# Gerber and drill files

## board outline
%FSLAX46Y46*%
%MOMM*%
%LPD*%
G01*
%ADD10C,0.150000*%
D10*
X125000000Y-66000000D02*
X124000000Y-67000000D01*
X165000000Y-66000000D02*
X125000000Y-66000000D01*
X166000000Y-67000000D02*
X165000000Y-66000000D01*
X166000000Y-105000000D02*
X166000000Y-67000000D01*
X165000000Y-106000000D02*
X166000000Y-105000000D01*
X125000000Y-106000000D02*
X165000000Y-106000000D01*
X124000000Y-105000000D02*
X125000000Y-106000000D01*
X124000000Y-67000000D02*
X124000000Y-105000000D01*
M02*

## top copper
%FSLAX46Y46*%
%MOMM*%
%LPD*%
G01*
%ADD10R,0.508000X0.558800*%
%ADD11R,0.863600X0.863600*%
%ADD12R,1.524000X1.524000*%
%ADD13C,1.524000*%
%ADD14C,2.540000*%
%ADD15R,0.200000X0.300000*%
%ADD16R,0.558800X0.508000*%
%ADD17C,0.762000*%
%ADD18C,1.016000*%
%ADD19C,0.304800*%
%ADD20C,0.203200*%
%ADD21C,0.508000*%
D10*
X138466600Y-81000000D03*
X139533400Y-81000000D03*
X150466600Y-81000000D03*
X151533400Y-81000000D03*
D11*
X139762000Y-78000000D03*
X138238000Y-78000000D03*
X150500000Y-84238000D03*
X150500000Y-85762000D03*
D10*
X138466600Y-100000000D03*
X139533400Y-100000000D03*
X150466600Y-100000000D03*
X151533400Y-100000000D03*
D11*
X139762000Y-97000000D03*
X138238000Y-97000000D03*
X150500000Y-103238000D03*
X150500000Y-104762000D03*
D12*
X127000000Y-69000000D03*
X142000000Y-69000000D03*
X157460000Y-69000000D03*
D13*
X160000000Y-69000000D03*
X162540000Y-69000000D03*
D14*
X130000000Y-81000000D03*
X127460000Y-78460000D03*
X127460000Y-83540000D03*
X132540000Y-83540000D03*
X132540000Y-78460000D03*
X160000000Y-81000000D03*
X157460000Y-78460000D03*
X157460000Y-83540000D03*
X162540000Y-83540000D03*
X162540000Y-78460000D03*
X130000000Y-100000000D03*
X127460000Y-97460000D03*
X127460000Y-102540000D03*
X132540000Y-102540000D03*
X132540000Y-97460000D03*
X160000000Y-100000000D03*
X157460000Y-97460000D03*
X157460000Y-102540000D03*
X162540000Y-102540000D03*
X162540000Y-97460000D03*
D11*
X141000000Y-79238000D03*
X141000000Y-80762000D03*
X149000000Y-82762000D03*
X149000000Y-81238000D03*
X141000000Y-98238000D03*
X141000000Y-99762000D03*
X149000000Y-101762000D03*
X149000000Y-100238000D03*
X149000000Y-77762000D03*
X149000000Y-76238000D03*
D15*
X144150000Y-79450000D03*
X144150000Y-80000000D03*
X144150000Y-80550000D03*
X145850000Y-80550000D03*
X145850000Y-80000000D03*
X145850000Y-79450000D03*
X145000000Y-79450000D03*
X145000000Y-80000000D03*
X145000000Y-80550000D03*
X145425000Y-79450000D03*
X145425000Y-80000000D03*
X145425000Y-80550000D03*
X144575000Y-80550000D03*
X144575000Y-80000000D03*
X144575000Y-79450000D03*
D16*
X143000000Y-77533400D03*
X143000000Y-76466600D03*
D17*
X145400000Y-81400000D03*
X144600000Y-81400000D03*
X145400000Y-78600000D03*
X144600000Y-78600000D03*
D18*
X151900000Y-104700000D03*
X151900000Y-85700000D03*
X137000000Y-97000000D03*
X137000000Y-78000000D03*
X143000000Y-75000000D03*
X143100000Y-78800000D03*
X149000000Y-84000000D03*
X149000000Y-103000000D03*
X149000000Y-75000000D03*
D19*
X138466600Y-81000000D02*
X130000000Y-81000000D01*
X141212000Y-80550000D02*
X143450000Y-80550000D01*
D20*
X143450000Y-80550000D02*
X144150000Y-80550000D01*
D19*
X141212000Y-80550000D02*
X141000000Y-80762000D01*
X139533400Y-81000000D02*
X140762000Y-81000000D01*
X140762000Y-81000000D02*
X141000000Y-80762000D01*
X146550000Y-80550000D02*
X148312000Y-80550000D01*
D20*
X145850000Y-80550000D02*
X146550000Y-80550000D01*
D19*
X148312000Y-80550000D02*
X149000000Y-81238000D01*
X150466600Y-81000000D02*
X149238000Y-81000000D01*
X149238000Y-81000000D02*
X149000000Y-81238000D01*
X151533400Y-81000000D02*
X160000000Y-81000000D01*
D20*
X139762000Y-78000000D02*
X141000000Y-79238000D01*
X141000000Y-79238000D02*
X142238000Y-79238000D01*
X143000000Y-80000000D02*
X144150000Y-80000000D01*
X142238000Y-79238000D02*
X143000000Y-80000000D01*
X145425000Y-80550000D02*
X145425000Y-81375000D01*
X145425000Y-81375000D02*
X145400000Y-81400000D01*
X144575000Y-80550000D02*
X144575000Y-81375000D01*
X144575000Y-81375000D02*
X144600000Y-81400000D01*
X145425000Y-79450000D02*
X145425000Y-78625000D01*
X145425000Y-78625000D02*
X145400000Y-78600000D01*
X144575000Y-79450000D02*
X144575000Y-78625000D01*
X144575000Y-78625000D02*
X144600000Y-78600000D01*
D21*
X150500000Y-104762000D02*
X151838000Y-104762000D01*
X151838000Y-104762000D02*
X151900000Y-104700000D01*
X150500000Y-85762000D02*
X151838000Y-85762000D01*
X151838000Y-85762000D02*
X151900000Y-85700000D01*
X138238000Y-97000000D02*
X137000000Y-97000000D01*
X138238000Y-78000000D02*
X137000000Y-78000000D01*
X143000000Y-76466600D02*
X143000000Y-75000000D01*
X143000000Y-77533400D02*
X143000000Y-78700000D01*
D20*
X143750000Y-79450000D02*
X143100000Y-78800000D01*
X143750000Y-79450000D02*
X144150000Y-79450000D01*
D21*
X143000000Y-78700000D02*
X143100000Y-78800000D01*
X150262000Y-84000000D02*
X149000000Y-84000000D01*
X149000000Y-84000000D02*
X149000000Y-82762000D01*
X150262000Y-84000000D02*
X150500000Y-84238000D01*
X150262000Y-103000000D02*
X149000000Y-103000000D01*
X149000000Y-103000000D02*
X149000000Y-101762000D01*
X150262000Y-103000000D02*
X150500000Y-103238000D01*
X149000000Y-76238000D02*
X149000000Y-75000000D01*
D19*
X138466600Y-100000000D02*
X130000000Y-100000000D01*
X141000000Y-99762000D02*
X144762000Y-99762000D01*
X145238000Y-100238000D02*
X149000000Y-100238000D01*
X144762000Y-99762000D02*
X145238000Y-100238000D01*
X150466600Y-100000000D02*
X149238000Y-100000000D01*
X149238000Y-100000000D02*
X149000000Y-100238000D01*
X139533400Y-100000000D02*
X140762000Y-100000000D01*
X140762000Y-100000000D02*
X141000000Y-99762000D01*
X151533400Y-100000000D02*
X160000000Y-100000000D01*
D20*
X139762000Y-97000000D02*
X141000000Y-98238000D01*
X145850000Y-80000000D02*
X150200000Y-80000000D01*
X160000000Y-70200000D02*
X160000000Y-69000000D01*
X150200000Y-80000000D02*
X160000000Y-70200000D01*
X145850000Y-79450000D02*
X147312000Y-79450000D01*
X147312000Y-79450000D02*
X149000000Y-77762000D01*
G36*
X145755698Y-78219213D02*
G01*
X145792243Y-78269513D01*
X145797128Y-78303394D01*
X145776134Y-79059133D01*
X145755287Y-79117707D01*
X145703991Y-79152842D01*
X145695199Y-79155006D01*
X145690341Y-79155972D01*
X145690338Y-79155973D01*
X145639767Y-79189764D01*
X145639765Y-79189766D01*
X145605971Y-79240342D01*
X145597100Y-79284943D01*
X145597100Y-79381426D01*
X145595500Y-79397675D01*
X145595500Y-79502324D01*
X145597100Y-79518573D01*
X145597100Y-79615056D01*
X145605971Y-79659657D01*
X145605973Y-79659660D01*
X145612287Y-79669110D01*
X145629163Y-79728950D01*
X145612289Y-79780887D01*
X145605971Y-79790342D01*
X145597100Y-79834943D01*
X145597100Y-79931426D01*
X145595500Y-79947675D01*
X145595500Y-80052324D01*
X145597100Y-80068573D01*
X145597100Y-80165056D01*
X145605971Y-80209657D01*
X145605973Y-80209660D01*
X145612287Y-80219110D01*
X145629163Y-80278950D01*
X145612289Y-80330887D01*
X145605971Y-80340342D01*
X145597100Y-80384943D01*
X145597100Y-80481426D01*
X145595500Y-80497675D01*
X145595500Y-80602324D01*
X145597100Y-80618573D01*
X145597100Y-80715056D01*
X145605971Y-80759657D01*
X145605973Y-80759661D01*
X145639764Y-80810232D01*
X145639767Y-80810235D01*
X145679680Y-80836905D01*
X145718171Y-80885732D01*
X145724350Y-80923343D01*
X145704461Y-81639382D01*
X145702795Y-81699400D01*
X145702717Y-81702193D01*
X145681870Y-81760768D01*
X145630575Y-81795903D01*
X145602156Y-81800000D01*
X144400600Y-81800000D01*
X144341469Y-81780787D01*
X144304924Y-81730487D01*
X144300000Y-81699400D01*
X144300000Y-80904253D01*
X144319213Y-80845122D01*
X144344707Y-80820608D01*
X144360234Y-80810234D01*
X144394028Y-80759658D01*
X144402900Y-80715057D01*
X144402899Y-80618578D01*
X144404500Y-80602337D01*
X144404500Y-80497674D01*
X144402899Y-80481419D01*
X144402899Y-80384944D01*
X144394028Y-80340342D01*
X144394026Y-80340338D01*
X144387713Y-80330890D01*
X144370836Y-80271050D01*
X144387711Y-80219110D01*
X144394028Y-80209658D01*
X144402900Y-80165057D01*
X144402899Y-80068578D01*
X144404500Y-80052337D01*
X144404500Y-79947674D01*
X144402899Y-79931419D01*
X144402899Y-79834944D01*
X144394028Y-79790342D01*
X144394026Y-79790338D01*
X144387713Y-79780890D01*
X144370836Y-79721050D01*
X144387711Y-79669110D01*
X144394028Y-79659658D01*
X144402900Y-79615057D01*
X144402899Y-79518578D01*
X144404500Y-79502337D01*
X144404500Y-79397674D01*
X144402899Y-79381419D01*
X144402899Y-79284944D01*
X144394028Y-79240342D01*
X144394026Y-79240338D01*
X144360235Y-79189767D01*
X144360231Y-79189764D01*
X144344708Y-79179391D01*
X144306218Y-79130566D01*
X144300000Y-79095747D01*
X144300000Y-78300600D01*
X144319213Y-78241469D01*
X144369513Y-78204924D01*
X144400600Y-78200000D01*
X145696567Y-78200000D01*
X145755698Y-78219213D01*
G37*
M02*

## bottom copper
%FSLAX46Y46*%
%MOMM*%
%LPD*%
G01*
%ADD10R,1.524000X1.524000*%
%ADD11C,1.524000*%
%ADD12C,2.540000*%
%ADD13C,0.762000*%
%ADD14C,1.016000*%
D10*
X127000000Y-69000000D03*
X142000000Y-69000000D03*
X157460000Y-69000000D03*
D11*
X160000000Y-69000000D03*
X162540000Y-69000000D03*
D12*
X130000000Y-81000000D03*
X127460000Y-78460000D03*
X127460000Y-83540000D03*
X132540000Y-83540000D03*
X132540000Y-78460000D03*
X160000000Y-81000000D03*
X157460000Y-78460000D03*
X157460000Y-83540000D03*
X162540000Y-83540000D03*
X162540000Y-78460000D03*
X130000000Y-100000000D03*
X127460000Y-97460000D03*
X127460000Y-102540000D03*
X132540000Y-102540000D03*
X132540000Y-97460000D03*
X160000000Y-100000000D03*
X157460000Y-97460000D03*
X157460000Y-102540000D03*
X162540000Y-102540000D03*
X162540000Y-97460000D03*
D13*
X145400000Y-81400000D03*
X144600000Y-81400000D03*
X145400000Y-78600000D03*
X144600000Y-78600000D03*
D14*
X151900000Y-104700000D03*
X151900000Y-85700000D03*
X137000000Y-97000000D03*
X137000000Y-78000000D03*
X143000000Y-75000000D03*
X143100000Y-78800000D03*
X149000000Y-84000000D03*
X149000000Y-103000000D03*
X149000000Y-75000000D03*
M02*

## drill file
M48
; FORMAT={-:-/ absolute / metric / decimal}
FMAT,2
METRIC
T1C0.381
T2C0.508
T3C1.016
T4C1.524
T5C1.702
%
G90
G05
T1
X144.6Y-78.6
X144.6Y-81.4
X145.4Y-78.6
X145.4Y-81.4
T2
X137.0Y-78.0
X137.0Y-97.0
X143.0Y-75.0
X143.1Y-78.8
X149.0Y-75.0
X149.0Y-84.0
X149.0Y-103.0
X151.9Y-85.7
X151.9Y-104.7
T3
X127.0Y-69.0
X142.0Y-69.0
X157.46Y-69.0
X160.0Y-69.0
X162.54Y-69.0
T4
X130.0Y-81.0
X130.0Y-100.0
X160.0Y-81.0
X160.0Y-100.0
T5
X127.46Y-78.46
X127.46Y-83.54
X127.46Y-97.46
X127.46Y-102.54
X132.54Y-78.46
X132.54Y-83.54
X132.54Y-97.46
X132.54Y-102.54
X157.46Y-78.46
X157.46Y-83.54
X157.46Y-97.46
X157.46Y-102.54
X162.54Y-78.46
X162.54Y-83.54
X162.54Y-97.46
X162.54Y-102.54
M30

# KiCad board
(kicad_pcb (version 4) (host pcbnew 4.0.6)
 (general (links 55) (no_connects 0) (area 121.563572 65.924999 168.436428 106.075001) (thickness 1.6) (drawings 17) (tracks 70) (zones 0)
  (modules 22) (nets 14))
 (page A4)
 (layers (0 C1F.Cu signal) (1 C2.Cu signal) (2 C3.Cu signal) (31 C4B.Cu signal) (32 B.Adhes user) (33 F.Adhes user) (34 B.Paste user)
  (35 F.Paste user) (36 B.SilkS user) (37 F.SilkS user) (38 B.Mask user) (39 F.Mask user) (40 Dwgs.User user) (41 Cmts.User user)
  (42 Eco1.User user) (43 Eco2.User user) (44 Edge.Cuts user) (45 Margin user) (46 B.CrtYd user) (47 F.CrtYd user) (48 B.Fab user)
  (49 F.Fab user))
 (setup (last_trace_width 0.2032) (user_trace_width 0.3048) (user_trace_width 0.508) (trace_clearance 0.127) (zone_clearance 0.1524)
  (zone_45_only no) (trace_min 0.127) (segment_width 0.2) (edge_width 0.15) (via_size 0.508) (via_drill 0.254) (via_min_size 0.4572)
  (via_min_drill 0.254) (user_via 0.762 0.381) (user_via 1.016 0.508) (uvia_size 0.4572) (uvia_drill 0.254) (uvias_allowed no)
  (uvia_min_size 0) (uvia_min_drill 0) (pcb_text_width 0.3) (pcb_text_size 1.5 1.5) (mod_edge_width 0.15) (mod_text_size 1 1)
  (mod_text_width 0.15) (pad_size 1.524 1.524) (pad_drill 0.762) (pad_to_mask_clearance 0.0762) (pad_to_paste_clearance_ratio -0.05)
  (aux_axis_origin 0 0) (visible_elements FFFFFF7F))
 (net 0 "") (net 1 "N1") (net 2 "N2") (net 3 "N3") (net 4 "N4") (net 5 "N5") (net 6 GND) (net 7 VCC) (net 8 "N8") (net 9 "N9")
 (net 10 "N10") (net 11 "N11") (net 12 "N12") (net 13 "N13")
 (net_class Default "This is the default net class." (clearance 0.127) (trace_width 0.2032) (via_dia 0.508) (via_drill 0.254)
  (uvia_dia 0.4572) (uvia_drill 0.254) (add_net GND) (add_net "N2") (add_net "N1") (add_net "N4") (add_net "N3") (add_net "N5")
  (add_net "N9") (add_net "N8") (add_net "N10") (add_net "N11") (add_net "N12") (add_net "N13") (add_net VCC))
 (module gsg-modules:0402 (layer C1F.Cu) (at 139 81 180) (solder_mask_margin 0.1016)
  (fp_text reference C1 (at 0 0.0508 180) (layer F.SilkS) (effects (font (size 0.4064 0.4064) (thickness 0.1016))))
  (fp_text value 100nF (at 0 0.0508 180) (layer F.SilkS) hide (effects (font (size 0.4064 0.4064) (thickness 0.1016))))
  (pad 2 smd rect (at 0.5334 0 180) (size 0.508 0.5588) (layers C1F.Cu F.Paste F.Mask) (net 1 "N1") (solder_mask_margin 0.1016))
  (pad 1 smd rect (at -0.5334 0 180) (size 0.508 0.5588) (layers C1F.Cu F.Paste F.Mask) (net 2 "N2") (solder_mask_margin 0.1016)))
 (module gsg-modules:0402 (layer C1F.Cu) (at 151 81 180) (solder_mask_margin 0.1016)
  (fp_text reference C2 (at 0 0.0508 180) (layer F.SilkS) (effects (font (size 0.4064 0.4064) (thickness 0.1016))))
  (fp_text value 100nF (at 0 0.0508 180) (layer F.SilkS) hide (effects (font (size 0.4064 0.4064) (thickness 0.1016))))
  (pad 2 smd rect (at 0.5334 0 180) (size 0.508 0.5588) (layers C1F.Cu F.Paste F.Mask) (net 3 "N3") (solder_mask_margin 0.1016))
  (pad 1 smd rect (at -0.5334 0 180) (size 0.508 0.5588) (layers C1F.Cu F.Paste F.Mask) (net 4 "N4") (solder_mask_margin 0.1016)))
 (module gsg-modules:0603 (layer C1F.Cu) (at 139 78) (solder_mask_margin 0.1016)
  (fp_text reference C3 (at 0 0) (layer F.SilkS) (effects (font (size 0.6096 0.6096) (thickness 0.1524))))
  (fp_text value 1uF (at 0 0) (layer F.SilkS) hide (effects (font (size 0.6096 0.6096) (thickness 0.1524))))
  (pad 2 smd rect (at 0.762 0) (size 0.8636 0.8636) (layers C1F.Cu F.Paste F.Mask) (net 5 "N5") (solder_mask_margin 0.1016)
   (clearance 0.1778))
  (pad 1 smd rect (at -0.762 0) (size 0.8636 0.8636) (layers C1F.Cu F.Paste F.Mask) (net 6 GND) (solder_mask_margin 0.1016)
   (clearance 0.1778)))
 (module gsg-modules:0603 (layer C1F.Cu) (at 150.5 85 90) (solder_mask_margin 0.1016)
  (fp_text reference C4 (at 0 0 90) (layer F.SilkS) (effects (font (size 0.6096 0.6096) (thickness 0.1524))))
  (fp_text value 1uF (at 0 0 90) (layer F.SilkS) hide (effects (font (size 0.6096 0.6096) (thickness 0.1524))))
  (pad 2 smd rect (at 0.762 0 90) (size 0.8636 0.8636) (layers C1F.Cu F.Paste F.Mask) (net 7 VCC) (solder_mask_margin 0.1016)
   (clearance 0.1778))
  (pad 1 smd rect (at -0.762 0 90) (size 0.8636 0.8636) (layers C1F.Cu F.Paste F.Mask) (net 6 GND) (solder_mask_margin 0.1016)
   (clearance 0.1778)))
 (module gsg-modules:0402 (layer C1F.Cu) (at 139 100 180) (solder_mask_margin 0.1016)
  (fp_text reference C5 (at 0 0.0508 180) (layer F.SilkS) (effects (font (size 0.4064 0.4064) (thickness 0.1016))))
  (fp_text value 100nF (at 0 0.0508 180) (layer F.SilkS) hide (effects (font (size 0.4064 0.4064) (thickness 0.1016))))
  (pad 2 smd rect (at 0.5334 0 180) (size 0.508 0.5588) (layers C1F.Cu F.Paste F.Mask) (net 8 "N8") (solder_mask_margin 0.1016))
  (pad 1 smd rect (at -0.5334 0 180) (size 0.508 0.5588) (layers C1F.Cu F.Paste F.Mask) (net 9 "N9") (solder_mask_margin 0.1016)))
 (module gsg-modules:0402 (layer C1F.Cu) (at 151 100 180) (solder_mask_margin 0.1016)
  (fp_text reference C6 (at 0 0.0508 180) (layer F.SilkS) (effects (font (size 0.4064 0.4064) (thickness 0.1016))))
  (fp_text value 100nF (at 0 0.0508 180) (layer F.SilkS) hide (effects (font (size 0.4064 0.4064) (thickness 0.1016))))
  (pad 2 smd rect (at 0.5334 0 180) (size 0.508 0.5588) (layers C1F.Cu F.Paste F.Mask) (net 9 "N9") (solder_mask_margin 0.1016))
  (pad 1 smd rect (at -0.5334 0 180) (size 0.508 0.5588) (layers C1F.Cu F.Paste F.Mask) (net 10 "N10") (solder_mask_margin 0.1016)))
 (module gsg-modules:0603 (layer C1F.Cu) (at 139 97) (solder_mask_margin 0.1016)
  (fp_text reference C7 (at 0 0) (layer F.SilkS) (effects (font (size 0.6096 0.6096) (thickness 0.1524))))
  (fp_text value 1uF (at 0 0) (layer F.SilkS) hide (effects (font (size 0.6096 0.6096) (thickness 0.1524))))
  (pad 2 smd rect (at 0.762 0) (size 0.8636 0.8636) (layers C1F.Cu F.Paste F.Mask) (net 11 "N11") (solder_mask_margin 0.1016)
   (clearance 0.1778))
  (pad 1 smd rect (at -0.762 0) (size 0.8636 0.8636) (layers C1F.Cu F.Paste F.Mask) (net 6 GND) (solder_mask_margin 0.1016)
   (clearance 0.1778)))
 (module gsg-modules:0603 (layer C1F.Cu) (at 150.5 104 90) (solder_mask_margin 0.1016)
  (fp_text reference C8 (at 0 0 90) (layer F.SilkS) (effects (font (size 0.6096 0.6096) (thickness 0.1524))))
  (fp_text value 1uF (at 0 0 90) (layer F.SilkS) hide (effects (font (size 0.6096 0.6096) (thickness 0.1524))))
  (pad 2 smd rect (at 0.762 0 90) (size 0.8636 0.8636) (layers C1F.Cu F.Paste F.Mask) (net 7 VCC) (solder_mask_margin 0.1016)
   (clearance 0.1778))
  (pad 1 smd rect (at -0.762 0 90) (size 0.8636 0.8636) (layers C1F.Cu F.Paste F.Mask) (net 6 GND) (solder_mask_margin 0.1016)
   (clearance 0.1778)))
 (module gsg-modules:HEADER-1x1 (layer C1F.Cu) (at 127 69)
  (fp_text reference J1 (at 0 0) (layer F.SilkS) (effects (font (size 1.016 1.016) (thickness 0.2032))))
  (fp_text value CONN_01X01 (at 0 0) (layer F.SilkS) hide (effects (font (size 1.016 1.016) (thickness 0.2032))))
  (pad 1 thru_hole rect (at 0 0) (size 1.524 1.524) (drill 1.016) (layers *.Cu *.Mask F.SilkS) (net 7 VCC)))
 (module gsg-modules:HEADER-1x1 (layer C1F.Cu) (at 142 69)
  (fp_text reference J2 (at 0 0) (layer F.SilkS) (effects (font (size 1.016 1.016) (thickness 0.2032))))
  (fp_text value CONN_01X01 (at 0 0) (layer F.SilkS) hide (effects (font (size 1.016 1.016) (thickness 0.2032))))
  (pad 1 thru_hole rect (at 0 0) (size 1.524 1.524) (drill 1.016) (layers *.Cu *.Mask F.SilkS) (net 6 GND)))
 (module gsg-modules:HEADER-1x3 (layer C1F.Cu) (at 160 69)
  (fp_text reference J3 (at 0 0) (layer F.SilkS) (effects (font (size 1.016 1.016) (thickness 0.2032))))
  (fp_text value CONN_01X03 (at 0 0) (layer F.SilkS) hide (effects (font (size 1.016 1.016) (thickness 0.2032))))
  (pad 1 thru_hole rect (at -2.54 0) (size 1.524 1.524) (drill 1.016) (layers *.Cu *.Mask F.SilkS) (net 7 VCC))
  (pad 2 thru_hole circle (at 0 0) (size 1.524 1.524) (drill 1.016) (layers *.Cu *.Mask F.SilkS) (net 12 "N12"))
  (pad 3 thru_hole circle (at 2.54 0) (size 1.524 1.524) (drill 1.016) (layers *.Cu *.Mask F.SilkS) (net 6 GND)))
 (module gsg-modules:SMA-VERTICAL (layer C1F.Cu) (at 130 81)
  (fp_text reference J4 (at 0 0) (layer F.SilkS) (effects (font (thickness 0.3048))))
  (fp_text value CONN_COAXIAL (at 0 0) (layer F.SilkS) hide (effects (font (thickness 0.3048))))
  (pad 1 thru_hole circle (at 0 0) (size 2.54 2.54) (drill 1.524) (layers *.Cu *.Mask F.SilkS) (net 1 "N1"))
  (pad 2 thru_hole circle (at -2.54 -2.54) (size 2.54 2.54) (drill 1.7018) (layers *.Cu *.Mask F.SilkS) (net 6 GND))
  (pad 2 thru_hole circle (at -2.54 2.54) (size 2.54 2.54) (drill 1.7018) (layers *.Cu *.Mask F.SilkS) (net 6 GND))
  (pad 2 thru_hole circle (at 2.54 2.54) (size 2.54 2.54) (drill 1.7018) (layers *.Cu *.Mask F.SilkS) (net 6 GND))
  (pad 2 thru_hole circle (at 2.54 -2.54) (size 2.54 2.54) (drill 1.7018) (layers *.Cu *.Mask F.SilkS) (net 6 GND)))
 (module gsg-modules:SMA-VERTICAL (layer C1F.Cu) (at 160 81)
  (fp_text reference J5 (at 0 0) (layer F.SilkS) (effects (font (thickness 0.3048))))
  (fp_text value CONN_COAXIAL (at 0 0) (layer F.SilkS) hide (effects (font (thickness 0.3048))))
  (pad 1 thru_hole circle (at 0 0) (size 2.54 2.54) (drill 1.524) (layers *.Cu *.Mask F.SilkS) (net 4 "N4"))
  (pad 2 thru_hole circle (at -2.54 -2.54) (size 2.54 2.54) (drill 1.7018) (layers *.Cu *.Mask F.SilkS) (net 6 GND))
  (pad 2 thru_hole circle (at -2.54 2.54) (size 2.54 2.54) (drill 1.7018) (layers *.Cu *.Mask F.SilkS) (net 6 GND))
  (pad 2 thru_hole circle (at 2.54 2.54) (size 2.54 2.54) (drill 1.7018) (layers *.Cu *.Mask F.SilkS) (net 6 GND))
  (pad 2 thru_hole circle (at 2.54 -2.54) (size 2.54 2.54) (drill 1.7018) (layers *.Cu *.Mask F.SilkS) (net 6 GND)))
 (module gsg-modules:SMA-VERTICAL (layer C1F.Cu) (at 130 100)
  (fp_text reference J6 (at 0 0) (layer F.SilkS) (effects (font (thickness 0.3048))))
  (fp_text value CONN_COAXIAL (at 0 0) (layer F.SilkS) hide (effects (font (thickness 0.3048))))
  (pad 1 thru_hole circle (at 0 0) (size 2.54 2.54) (drill 1.524) (layers *.Cu *.Mask F.SilkS) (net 8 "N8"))
  (pad 2 thru_hole circle (at -2.54 -2.54) (size 2.54 2.54) (drill 1.7018) (layers *.Cu *.Mask F.SilkS) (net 6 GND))
  (pad 2 thru_hole circle (at -2.54 2.54) (size 2.54 2.54) (drill 1.7018) (layers *.Cu *.Mask F.SilkS) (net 6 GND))
  (pad 2 thru_hole circle (at 2.54 2.54) (size 2.54 2.54) (drill 1.7018) (layers *.Cu *.Mask F.SilkS) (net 6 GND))
  (pad 2 thru_hole circle (at 2.54 -2.54) (size 2.54 2.54) (drill 1.7018) (layers *.Cu *.Mask F.SilkS) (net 6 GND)))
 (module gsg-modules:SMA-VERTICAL (layer C1F.Cu) (at 160 100)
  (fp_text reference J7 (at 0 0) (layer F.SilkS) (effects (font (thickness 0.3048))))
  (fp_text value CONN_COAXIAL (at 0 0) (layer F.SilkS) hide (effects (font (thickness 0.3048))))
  (pad 1 thru_hole circle (at 0 0) (size 2.54 2.54) (drill 1.524) (layers *.Cu *.Mask F.SilkS) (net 10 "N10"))
  (pad 2 thru_hole circle (at -2.54 -2.54) (size 2.54 2.54) (drill 1.7018) (layers *.Cu *.Mask F.SilkS) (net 6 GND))
  (pad 2 thru_hole circle (at -2.54 2.54) (size 2.54 2.54) (drill 1.7018) (layers *.Cu *.Mask F.SilkS) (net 6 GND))
  (pad 2 thru_hole circle (at 2.54 2.54) (size 2.54 2.54) (drill 1.7018) (layers *.Cu *.Mask F.SilkS) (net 6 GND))
  (pad 2 thru_hole circle (at 2.54 -2.54) (size 2.54 2.54) (drill 1.7018) (layers *.Cu *.Mask F.SilkS) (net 6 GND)))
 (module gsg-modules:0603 (layer C1F.Cu) (at 141 80 90) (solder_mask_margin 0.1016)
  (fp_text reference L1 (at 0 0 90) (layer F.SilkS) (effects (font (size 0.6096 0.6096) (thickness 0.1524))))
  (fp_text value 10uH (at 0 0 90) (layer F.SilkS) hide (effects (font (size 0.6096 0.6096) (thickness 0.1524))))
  (pad 2 smd rect (at 0.762 0 90) (size 0.8636 0.8636) (layers C1F.Cu F.Paste F.Mask) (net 5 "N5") (solder_mask_margin 0.1016)
   (clearance 0.1778))
  (pad 1 smd rect (at -0.762 0 90) (size 0.8636 0.8636) (layers C1F.Cu F.Paste F.Mask) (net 2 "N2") (solder_mask_margin 0.1016)
   (clearance 0.1778)))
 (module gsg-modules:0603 (layer C1F.Cu) (at 149 82 270) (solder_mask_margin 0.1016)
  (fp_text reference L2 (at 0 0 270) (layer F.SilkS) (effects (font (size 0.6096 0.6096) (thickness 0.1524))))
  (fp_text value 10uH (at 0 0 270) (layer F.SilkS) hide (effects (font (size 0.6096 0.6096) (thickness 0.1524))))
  (pad 2 smd rect (at 0.762 0 270) (size 0.8636 0.8636) (layers C1F.Cu F.Paste F.Mask) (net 7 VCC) (solder_mask_margin 0.1016)
   (clearance 0.1778))
  (pad 1 smd rect (at -0.762 0 270) (size 0.8636 0.8636) (layers C1F.Cu F.Paste F.Mask) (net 3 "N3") (solder_mask_margin 0.1016)
   (clearance 0.1778)))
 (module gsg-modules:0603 (layer C1F.Cu) (at 141 99 90) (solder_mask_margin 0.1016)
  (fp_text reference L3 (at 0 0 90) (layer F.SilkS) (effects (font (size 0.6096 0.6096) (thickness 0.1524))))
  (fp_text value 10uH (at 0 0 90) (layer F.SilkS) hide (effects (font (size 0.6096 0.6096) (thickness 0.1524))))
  (pad 2 smd rect (at 0.762 0 90) (size 0.8636 0.8636) (layers C1F.Cu F.Paste F.Mask) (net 11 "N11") (solder_mask_margin 0.1016)
   (clearance 0.1778))
  (pad 1 smd rect (at -0.762 0 90) (size 0.8636 0.8636) (layers C1F.Cu F.Paste F.Mask) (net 9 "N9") (solder_mask_margin 0.1016)
   (clearance 0.1778)))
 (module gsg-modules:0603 (layer C1F.Cu) (at 149 101 270) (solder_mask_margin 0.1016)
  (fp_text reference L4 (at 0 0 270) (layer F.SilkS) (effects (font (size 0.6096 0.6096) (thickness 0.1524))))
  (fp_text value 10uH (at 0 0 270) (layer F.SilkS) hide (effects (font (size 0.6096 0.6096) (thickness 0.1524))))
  (pad 2 smd rect (at 0.762 0 270) (size 0.8636 0.8636) (layers C1F.Cu F.Paste F.Mask) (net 7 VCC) (solder_mask_margin 0.1016)
   (clearance 0.1778))
  (pad 1 smd rect (at -0.762 0 270) (size 0.8636 0.8636) (layers C1F.Cu F.Paste F.Mask) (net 9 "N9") (solder_mask_margin 0.1016)
   (clearance 0.1778)))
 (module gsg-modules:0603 (layer C1F.Cu) (at 149 77 270) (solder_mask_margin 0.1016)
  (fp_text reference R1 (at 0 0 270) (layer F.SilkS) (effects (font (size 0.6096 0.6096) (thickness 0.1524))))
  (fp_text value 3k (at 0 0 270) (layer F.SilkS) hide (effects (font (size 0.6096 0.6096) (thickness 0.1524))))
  (pad 2 smd rect (at 0.762 0 270) (size 0.8636 0.8636) (layers C1F.Cu F.Paste F.Mask) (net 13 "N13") (solder_mask_margin 0.1016)
   (clearance 0.1778))
  (pad 1 smd rect (at -0.762 0 270) (size 0.8636 0.8636) (layers C1F.Cu F.Paste F.Mask) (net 7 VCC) (solder_mask_margin 0.1016)
   (clearance 0.1778)))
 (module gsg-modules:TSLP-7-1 (layer C1F.Cu) (at 145 80 270)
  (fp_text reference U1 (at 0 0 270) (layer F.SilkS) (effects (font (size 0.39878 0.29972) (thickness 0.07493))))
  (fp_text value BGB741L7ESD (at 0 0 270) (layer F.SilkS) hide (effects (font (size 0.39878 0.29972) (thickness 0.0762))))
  (pad 1 smd rect (at -0.55 0.85 270) (size 0.3 0.2) (layers C1F.Cu F.Paste F.Mask) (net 7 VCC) (die_length 3.40614))
  (pad 2 smd rect (at 0 0.85 270) (size 0.3 0.2) (layers C1F.Cu F.Paste F.Mask) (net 5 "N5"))
  (pad 3 smd rect (at 0.55 0.85 270) (size 0.3 0.2) (layers C1F.Cu F.Paste F.Mask) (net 2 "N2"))
  (pad 4 smd rect (at 0.55 -0.85 270) (size 0.3 0.2) (layers C1F.Cu F.Paste F.Mask) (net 3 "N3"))
  (pad 5 smd rect (at 0 -0.85 270) (size 0.3 0.2) (layers C1F.Cu F.Paste F.Mask) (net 12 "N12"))
  (pad 6 smd rect (at -0.55 -0.85 270) (size 0.3 0.2) (layers C1F.Cu F.Paste F.Mask) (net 13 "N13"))
  (pad 7 smd rect (at -0.55 0 270) (size 0.3 0.2) (layers C1F.Cu F.Paste F.Mask) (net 6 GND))
  (pad 7 smd rect (at 0 0 270) (size 0.3 0.2) (layers C1F.Cu F.Paste F.Mask) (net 6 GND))
  (pad 7 smd rect (at 0.55 0 270) (size 0.3 0.2) (layers C1F.Cu F.Paste F.Mask) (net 6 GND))
  (pad 7 smd rect (at -0.55 -0.425 270) (size 0.3 0.2) (layers C1F.Cu F.Paste F.Mask) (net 6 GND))
  (pad 7 smd rect (at 0 -0.425 270) (size 0.3 0.2) (layers C1F.Cu F.Paste F.Mask) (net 6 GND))
  (pad 7 smd rect (at 0.55 -0.425 270) (size 0.3 0.2) (layers C1F.Cu F.Paste F.Mask) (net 6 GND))
  (pad 7 smd rect (at 0.55 0.425 270) (size 0.3 0.2) (layers C1F.Cu F.Paste F.Mask) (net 6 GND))
  (pad 7 smd rect (at 0 0.425 270) (size 0.3 0.2) (layers C1F.Cu F.Paste F.Mask) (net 6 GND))
  (pad 7 smd rect (at -0.55 0.425 270) (size 0.3 0.2) (layers C1F.Cu F.Paste F.Mask) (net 6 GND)))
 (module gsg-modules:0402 (layer C1F.Cu) (at 143 77 270) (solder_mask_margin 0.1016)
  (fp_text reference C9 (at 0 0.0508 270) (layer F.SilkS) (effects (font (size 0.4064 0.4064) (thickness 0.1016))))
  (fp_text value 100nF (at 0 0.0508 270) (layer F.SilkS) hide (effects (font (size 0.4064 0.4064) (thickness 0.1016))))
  (pad 2 smd rect (at 0.5334 0 270) (size 0.508 0.5588) (layers C1F.Cu F.Paste F.Mask) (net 7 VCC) (solder_mask_margin 0.1016))
  (pad 1 smd rect (at -0.5334 0 270) (size 0.508 0.5588) (layers C1F.Cu F.Paste F.Mask) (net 6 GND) (solder_mask_margin 0.1016)))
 (gr_line (start 125 66) (end 124 67) (angle 90) (layer Edge.Cuts) (width 0.15))
 (gr_line (start 165 66) (end 125 66) (angle 90) (layer Edge.Cuts) (width 0.15))
 (gr_line (start 166 67) (end 165 66) (angle 90) (layer Edge.Cuts) (width 0.15))
 (gr_line (start 166 105) (end 166 67) (angle 90) (layer Edge.Cuts) (width 0.15))
 (gr_line (start 165 106) (end 166 105) (angle 90) (layer Edge.Cuts) (width 0.15))
 (gr_line (start 125 106) (end 165 106) (angle 90) (layer Edge.Cuts) (width 0.15))
 (gr_line (start 124 105) (end 125 106) (angle 90) (layer Edge.Cuts) (width 0.15))
 (gr_line (start 124 67) (end 124 105) (angle 90) (layer Edge.Cuts) (width 0.15))
 (segment (start 138.4666 81) (end 130 81) (width 0.3048) (layer C1F.Cu) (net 1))
 (segment (start 141.212 80.55) (end 143.45 80.55) (width 0.3048) (layer C1F.Cu) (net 2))
 (segment (start 143.45 80.55) (end 144.15 80.55) (width 0.2032) (layer C1F.Cu) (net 2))
 (segment (start 141.212 80.55) (end 141 80.762) (width 0.3048) (layer C1F.Cu) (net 2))
 (segment (start 139.5334 81) (end 140.762 81) (width 0.3048) (layer C1F.Cu) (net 2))
 (segment (start 140.762 81) (end 141 80.762) (width 0.3048) (layer C1F.Cu) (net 2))
 (segment (start 146.55 80.55) (end 148.312 80.55) (width 0.3048) (layer C1F.Cu) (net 3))
 (segment (start 145.85 80.55) (end 146.55 80.55) (width 0.2032) (layer C1F.Cu) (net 3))
 (segment (start 148.312 80.55) (end 149 81.238) (width 0.3048) (layer C1F.Cu) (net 3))
 (segment (start 150.4666 81) (end 149.238 81) (width 0.3048) (layer C1F.Cu) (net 3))
 (segment (start 149.238 81) (end 149 81.238) (width 0.3048) (layer C1F.Cu) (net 3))
 (segment (start 151.5334 81) (end 160 81) (width 0.3048) (layer C1F.Cu) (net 4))
 (segment (start 139.762 78) (end 141 79.238) (width 0.2032) (layer C1F.Cu) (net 5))
 (segment (start 141 79.238) (end 142.238 79.238) (width 0.2032) (layer C1F.Cu) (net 5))
 (segment (start 143 80) (end 144.15 80) (width 0.2032) (layer C1F.Cu) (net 5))
 (segment (start 142.238 79.238) (end 143 80) (width 0.2032) (layer C1F.Cu) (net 5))
 (segment (start 145.425 80.55) (end 145.425 81.375) (width 0.2032) (layer C1F.Cu) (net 6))
 (via (at 145.4 81.4) (size 0.762) (drill 0.381) (layers C1F.Cu C4B.Cu) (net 6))
 (segment (start 145.425 81.375) (end 145.4 81.4) (width 0.2032) (layer C1F.Cu) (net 6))
 (segment (start 144.575 80.55) (end 144.575 81.375) (width 0.2032) (layer C1F.Cu) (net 6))
 (via (at 144.6 81.4) (size 0.762) (drill 0.381) (layers C1F.Cu C4B.Cu) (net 6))
 (segment (start 144.575 81.375) (end 144.6 81.4) (width 0.2032) (layer C1F.Cu) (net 6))
 (segment (start 145.425 79.45) (end 145.425 78.625) (width 0.2032) (layer C1F.Cu) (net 6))
 (via (at 145.4 78.6) (size 0.762) (drill 0.381) (layers C1F.Cu C4B.Cu) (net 6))
 (segment (start 145.425 78.625) (end 145.4 78.6) (width 0.2032) (layer C1F.Cu) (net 6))
 (segment (start 144.575 79.45) (end 144.575 78.625) (width 0.2032) (layer C1F.Cu) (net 6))
 (via (at 144.6 78.6) (size 0.762) (drill 0.381) (layers C1F.Cu C4B.Cu) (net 6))
 (segment (start 144.575 78.625) (end 144.6 78.6) (width 0.2032) (layer C1F.Cu) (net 6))
 (segment (start 150.5 104.762) (end 151.838 104.762) (width 0.508) (layer C1F.Cu) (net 6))
 (via (at 151.9 104.7) (size 1.016) (drill 0.508) (layers C1F.Cu C4B.Cu) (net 6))
 (segment (start 151.838 104.762) (end 151.9 104.7) (width 0.508) (layer C1F.Cu) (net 6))
 (segment (start 150.5 85.762) (end 151.838 85.762) (width 0.508) (layer C1F.Cu) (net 6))
 (via (at 151.9 85.7) (size 1.016) (drill 0.508) (layers C1F.Cu C4B.Cu) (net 6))
 (segment (start 151.838 85.762) (end 151.9 85.7) (width 0.508) (layer C1F.Cu) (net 6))
 (segment (start 138.238 97) (end 137 97) (width 0.508) (layer C1F.Cu) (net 6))
 (via (at 137 97) (size 1.016) (drill 0.508) (layers C1F.Cu C4B.Cu) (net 6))
 (segment (start 138.238 78) (end 137 78) (width 0.508) (layer C1F.Cu) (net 6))
 (via (at 137 78) (size 1.016) (drill 0.508) (layers C1F.Cu C4B.Cu) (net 6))
 (segment (start 143 76.4666) (end 143 75) (width 0.508) (layer C1F.Cu) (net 6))
 (via (at 143 75) (size 1.016) (drill 0.508) (layers C1F.Cu C4B.Cu) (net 6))
 (segment (start 143 77.5334) (end 143 78.7) (width 0.508) (layer C1F.Cu) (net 7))
 (segment (start 143.75 79.45) (end 143.1 78.8) (width 0.2032) (layer C1F.Cu) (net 7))
 (via (at 143.1 78.8) (size 1.016) (drill 0.508) (layers C1F.Cu C4B.Cu) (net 7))
 (segment (start 143.75 79.45) (end 144.15 79.45) (width 0.2032) (layer C1F.Cu) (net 7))
 (segment (start 143 78.7) (end 143.1 78.8) (width 0.508) (layer C1F.Cu) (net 7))
 (segment (start 150.262 84) (end 149 84) (width 0.508) (layer C1F.Cu) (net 7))
 (via (at 149 84) (size 1.016) (drill 0.508) (layers C1F.Cu C4B.Cu) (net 7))
 (segment (start 149 84) (end 149 82.762) (width 0.508) (layer C1F.Cu) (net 7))
 (segment (start 150.262 84) (end 150.5 84.238) (width 0.508) (layer C1F.Cu) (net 7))
 (segment (start 150.262 103) (end 149 103) (width 0.508) (layer C1F.Cu) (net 7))
 (via (at 149 103) (size 1.016) (drill 0.508) (layers C1F.Cu C4B.Cu) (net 7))
 (segment (start 149 103) (end 149 101.762) (width 0.508) (layer C1F.Cu) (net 7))
 (segment (start 150.262 103) (end 150.5 103.238) (width 0.508) (layer C1F.Cu) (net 7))
 (segment (start 149 76.238) (end 149 75) (width 0.508) (layer C1F.Cu) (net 7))
 (via (at 149 75) (size 1.016) (drill 0.508) (layers C1F.Cu C4B.Cu) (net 7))
 (segment (start 138.4666 100) (end 130 100) (width 0.3048) (layer C1F.Cu) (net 8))
 (segment (start 141 99.762) (end 144.762 99.762) (width 0.3048) (layer C1F.Cu) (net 9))
 (segment (start 145.238 100.238) (end 149 100.238) (width 0.3048) (layer C1F.Cu) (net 9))
 (segment (start 144.762 99.762) (end 145.238 100.238) (width 0.3048) (layer C1F.Cu) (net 9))
 (segment (start 150.4666 100) (end 149.238 100) (width 0.3048) (layer C1F.Cu) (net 9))
 (segment (start 149.238 100) (end 149 100.238) (width 0.3048) (layer C1F.Cu) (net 9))
 (segment (start 139.5334 100) (end 140.762 100) (width 0.3048) (layer C1F.Cu) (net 9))
 (segment (start 140.762 100) (end 141 99.762) (width 0.3048) (layer C1F.Cu) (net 9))
 (segment (start 151.5334 100) (end 160 100) (width 0.3048) (layer C1F.Cu) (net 10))
 (segment (start 139.762 97) (end 141 98.238) (width 0.2032) (layer C1F.Cu) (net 11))
 (segment (start 145.85 80) (end 150.2 80) (width 0.2032) (layer C1F.Cu) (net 12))
 (segment (start 160 70.2) (end 160 69) (width 0.2032) (layer C1F.Cu) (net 12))
 (segment (start 150.2 80) (end 160 70.2) (width 0.2032) (layer C1F.Cu) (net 12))
 (segment (start 145.85 79.45) (end 147.312 79.45) (width 0.2032) (layer C1F.Cu) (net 13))
 (segment (start 147.312 79.45) (end 149 77.762) (width 0.2032) (layer C1F.Cu) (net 13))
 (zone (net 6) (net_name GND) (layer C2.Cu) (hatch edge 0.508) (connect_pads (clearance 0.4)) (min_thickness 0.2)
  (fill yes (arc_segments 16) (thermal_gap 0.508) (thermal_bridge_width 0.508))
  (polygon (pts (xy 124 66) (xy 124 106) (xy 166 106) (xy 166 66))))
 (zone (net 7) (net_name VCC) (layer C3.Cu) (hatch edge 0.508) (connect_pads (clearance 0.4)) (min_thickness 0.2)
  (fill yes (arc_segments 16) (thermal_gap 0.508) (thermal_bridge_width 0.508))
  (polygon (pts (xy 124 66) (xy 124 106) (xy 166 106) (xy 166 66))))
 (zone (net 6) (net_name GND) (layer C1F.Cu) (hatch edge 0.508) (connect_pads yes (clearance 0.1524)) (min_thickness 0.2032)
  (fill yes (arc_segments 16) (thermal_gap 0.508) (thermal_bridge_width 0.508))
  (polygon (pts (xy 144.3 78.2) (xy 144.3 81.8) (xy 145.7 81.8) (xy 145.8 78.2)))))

